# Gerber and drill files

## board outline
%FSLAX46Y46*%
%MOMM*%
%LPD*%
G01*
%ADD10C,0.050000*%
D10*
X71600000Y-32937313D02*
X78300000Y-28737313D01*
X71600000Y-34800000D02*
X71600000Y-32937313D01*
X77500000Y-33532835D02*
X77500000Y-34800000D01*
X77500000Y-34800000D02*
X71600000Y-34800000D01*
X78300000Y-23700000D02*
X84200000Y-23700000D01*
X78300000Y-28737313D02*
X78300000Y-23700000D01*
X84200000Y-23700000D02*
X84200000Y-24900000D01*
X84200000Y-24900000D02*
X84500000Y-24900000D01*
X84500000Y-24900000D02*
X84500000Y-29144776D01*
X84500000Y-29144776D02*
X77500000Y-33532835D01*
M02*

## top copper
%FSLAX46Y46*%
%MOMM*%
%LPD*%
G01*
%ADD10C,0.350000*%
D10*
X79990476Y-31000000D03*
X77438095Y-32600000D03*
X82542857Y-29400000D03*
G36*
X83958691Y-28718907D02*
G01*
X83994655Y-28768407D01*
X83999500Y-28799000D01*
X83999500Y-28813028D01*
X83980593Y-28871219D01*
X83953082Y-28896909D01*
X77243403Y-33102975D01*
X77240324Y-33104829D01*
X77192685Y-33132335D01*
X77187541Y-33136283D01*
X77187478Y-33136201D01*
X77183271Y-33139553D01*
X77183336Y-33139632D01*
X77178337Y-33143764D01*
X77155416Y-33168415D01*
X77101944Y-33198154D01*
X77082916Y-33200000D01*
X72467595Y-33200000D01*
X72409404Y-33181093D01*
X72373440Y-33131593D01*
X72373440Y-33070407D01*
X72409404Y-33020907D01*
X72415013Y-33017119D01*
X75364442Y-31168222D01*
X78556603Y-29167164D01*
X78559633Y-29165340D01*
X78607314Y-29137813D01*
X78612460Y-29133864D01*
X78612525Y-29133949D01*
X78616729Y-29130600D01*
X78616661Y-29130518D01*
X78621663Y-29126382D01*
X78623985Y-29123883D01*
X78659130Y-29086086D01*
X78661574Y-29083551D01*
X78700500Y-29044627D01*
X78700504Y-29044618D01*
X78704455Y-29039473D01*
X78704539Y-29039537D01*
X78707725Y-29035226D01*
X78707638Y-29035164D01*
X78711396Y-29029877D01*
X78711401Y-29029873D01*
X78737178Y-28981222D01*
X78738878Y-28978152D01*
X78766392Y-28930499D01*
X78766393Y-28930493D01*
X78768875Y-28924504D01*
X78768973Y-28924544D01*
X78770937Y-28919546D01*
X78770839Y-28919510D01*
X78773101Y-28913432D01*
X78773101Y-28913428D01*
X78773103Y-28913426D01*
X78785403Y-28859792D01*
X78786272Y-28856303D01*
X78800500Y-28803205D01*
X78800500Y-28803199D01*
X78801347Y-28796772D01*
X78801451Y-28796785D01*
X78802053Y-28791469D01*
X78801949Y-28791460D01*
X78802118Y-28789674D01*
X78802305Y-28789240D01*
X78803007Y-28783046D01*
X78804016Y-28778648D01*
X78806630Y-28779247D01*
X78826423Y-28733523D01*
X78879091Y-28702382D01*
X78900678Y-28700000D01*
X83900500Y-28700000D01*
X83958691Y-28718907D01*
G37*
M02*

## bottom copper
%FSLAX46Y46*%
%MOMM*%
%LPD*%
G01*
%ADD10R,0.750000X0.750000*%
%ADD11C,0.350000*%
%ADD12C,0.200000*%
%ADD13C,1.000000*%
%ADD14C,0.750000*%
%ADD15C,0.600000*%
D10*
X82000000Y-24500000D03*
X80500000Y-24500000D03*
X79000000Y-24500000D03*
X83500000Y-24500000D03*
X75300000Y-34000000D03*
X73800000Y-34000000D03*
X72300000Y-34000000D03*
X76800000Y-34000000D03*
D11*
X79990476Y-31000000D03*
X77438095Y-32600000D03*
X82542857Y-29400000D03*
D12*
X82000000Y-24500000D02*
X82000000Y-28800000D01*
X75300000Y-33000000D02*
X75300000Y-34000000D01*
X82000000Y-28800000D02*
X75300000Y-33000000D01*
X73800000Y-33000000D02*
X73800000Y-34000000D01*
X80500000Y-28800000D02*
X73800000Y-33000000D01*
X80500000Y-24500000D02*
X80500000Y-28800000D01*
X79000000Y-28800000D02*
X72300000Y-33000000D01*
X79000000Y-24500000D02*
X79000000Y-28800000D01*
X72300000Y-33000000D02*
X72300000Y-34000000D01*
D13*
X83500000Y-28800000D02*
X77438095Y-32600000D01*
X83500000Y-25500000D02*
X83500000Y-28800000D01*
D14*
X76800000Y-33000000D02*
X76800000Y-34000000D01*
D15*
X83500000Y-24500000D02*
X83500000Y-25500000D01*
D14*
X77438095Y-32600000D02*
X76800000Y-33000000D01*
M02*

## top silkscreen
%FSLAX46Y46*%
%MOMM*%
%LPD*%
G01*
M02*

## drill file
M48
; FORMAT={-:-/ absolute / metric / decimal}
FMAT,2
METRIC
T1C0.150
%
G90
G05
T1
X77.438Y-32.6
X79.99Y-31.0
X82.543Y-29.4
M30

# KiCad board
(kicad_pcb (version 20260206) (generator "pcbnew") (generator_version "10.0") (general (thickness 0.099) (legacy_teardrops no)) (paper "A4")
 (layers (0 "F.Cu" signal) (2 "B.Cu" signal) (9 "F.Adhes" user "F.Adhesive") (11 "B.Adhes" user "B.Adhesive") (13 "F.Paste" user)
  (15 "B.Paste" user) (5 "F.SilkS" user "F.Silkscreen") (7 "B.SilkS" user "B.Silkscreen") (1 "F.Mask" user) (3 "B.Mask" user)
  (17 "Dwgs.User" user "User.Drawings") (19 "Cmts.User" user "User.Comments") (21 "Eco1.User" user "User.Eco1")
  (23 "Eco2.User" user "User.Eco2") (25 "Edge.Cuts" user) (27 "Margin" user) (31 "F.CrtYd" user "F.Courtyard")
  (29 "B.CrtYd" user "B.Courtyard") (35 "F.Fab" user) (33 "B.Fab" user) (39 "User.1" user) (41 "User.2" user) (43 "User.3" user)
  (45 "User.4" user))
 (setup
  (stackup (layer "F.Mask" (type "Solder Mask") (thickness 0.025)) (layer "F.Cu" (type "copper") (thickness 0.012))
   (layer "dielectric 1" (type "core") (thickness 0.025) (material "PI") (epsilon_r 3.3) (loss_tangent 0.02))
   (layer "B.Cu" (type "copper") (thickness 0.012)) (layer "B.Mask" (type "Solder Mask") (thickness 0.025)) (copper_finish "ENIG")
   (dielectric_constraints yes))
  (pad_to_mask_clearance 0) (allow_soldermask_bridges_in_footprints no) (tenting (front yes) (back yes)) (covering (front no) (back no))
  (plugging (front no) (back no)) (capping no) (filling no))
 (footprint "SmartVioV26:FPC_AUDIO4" (layer "F.Cu") (at 0 0)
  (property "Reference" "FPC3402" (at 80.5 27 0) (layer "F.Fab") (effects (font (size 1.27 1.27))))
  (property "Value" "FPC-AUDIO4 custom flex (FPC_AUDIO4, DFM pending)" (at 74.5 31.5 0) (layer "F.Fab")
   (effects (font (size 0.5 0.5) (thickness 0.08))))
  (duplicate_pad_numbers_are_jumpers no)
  (pad "S1" smd rect (at 82 24.5) (size 0.75 0.75) (layers "B.Cu" "B.Mask") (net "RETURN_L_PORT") (solder_mask_margin 0.1)
   (thermal_bridge_angle 45))
  (pad "S2" smd rect (at 80.5 24.5) (size 0.75 0.75) (layers "B.Cu" "B.Mask") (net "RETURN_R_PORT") (solder_mask_margin 0.1)
   (thermal_bridge_angle 45))
  (pad "S3" smd rect (at 79 24.5) (size 0.75 0.75) (layers "B.Cu" "B.Mask") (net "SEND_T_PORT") (solder_mask_margin 0.1)
   (thermal_bridge_angle 45))
  (pad "S4" smd rect (at 83.5 24.5) (size 0.75 0.75) (layers "B.Cu" "B.Mask") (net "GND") (solder_mask_margin 0.1) (thermal_bridge_angle 45))
  (pad "T1" smd rect (at 75.3 34) (size 0.75 0.75) (layers "B.Cu" "B.Mask") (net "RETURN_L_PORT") (solder_mask_margin 0.1)
   (thermal_bridge_angle 45))
  (pad "T2" smd rect (at 73.8 34) (size 0.75 0.75) (layers "B.Cu" "B.Mask") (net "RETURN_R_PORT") (solder_mask_margin 0.1)
   (thermal_bridge_angle 45))
  (pad "T3" smd rect (at 72.3 34) (size 0.75 0.75) (layers "B.Cu" "B.Mask") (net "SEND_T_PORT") (solder_mask_margin 0.1)
   (thermal_bridge_angle 45))
  (pad "T4" smd rect (at 76.8 34) (size 0.75 0.75) (layers "B.Cu" "B.Mask") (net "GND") (solder_mask_margin 0.1) (thermal_bridge_angle 45)))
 (gr_line (start 71.6 32.937313) (end 78.3 28.737313) (stroke (width 0.05) (type default)) (layer "Edge.Cuts"))
 (gr_line (start 71.6 34.8) (end 71.6 32.937313) (stroke (width 0.05) (type default)) (layer "Edge.Cuts"))
 (gr_line (start 77.5 33.532835) (end 77.5 34.8) (stroke (width 0.05) (type default)) (layer "Edge.Cuts"))
 (gr_line (start 77.5 34.8) (end 71.6 34.8) (stroke (width 0.05) (type default)) (layer "Edge.Cuts"))
 (gr_line (start 78.3 23.7) (end 84.2 23.7) (stroke (width 0.05) (type default)) (layer "Edge.Cuts"))
 (gr_line (start 78.3 28.737313) (end 78.3 23.7) (stroke (width 0.05) (type default)) (layer "Edge.Cuts"))
 (gr_line (start 84.2 23.7) (end 84.2 24.9) (stroke (width 0.05) (type default)) (layer "Edge.Cuts"))
 (gr_line (start 84.2 24.9) (end 84.5 24.9) (stroke (width 0.05) (type default)) (layer "Edge.Cuts"))
 (gr_line (start 84.5 24.9) (end 84.5 29.144776) (stroke (width 0.05) (type default)) (layer "Edge.Cuts"))
 (gr_line (start 84.5 29.144776) (end 77.5 33.532835) (stroke (width 0.05) (type default)) (layer "Edge.Cuts"))
 (segment (start 82 24.5) (end 82 28.8) (width 0.2) (layer "B.Cu") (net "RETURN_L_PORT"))
 (segment (start 75.3 33) (end 75.3 34) (width 0.2) (layer "B.Cu") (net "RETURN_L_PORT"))
 (segment (start 82 28.8) (end 75.3 33) (width 0.2) (layer "B.Cu") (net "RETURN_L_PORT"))
 (segment (start 73.8 33) (end 73.8 34) (width 0.2) (layer "B.Cu") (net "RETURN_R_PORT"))
 (segment (start 80.5 28.8) (end 73.8 33) (width 0.2) (layer "B.Cu") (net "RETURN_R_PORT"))
 (segment (start 80.5 24.5) (end 80.5 28.8) (width 0.2) (layer "B.Cu") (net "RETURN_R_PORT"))
 (segment (start 79 28.8) (end 72.3 33) (width 0.2) (layer "B.Cu") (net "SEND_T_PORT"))
 (segment (start 79 24.5) (end 79 28.8) (width 0.2) (layer "B.Cu") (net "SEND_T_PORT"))
 (segment (start 72.3 33) (end 72.3 34) (width 0.2) (layer "B.Cu") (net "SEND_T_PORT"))
 (via (at 79.990476 31) (size 0.35) (drill 0.15) (layers "F.Cu" "B.Cu") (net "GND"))
 (via (at 77.438095 32.6) (size 0.35) (drill 0.15) (layers "F.Cu" "B.Cu") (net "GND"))
 (via (at 82.542857 29.4) (size 0.35) (drill 0.15) (layers "F.Cu" "B.Cu") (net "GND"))
 (segment (start 83.5 28.8) (end 77.438095 32.6) (width 1) (layer "B.Cu") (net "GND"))
 (segment (start 83.5 25.5) (end 83.5 28.8) (width 1) (layer "B.Cu") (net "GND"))
 (segment (start 76.8 33) (end 76.8 34) (width 0.75) (layer "B.Cu") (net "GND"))
 (segment (start 83.5 24.5) (end 83.5 25.5) (width 0.6) (layer "B.Cu") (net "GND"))
 (segment (start 77.438095 32.6) (end 76.8 33) (width 0.75) (layer "B.Cu") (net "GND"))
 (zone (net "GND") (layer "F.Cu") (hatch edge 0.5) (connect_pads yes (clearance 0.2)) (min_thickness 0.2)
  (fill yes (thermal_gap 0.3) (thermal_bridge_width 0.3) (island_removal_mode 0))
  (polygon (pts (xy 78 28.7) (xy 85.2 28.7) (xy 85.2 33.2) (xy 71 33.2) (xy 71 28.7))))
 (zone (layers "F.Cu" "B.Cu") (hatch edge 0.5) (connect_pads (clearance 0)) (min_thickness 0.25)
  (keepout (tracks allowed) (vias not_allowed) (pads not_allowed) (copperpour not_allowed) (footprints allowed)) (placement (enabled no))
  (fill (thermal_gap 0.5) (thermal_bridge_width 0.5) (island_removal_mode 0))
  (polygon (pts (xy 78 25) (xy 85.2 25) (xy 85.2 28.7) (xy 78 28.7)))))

